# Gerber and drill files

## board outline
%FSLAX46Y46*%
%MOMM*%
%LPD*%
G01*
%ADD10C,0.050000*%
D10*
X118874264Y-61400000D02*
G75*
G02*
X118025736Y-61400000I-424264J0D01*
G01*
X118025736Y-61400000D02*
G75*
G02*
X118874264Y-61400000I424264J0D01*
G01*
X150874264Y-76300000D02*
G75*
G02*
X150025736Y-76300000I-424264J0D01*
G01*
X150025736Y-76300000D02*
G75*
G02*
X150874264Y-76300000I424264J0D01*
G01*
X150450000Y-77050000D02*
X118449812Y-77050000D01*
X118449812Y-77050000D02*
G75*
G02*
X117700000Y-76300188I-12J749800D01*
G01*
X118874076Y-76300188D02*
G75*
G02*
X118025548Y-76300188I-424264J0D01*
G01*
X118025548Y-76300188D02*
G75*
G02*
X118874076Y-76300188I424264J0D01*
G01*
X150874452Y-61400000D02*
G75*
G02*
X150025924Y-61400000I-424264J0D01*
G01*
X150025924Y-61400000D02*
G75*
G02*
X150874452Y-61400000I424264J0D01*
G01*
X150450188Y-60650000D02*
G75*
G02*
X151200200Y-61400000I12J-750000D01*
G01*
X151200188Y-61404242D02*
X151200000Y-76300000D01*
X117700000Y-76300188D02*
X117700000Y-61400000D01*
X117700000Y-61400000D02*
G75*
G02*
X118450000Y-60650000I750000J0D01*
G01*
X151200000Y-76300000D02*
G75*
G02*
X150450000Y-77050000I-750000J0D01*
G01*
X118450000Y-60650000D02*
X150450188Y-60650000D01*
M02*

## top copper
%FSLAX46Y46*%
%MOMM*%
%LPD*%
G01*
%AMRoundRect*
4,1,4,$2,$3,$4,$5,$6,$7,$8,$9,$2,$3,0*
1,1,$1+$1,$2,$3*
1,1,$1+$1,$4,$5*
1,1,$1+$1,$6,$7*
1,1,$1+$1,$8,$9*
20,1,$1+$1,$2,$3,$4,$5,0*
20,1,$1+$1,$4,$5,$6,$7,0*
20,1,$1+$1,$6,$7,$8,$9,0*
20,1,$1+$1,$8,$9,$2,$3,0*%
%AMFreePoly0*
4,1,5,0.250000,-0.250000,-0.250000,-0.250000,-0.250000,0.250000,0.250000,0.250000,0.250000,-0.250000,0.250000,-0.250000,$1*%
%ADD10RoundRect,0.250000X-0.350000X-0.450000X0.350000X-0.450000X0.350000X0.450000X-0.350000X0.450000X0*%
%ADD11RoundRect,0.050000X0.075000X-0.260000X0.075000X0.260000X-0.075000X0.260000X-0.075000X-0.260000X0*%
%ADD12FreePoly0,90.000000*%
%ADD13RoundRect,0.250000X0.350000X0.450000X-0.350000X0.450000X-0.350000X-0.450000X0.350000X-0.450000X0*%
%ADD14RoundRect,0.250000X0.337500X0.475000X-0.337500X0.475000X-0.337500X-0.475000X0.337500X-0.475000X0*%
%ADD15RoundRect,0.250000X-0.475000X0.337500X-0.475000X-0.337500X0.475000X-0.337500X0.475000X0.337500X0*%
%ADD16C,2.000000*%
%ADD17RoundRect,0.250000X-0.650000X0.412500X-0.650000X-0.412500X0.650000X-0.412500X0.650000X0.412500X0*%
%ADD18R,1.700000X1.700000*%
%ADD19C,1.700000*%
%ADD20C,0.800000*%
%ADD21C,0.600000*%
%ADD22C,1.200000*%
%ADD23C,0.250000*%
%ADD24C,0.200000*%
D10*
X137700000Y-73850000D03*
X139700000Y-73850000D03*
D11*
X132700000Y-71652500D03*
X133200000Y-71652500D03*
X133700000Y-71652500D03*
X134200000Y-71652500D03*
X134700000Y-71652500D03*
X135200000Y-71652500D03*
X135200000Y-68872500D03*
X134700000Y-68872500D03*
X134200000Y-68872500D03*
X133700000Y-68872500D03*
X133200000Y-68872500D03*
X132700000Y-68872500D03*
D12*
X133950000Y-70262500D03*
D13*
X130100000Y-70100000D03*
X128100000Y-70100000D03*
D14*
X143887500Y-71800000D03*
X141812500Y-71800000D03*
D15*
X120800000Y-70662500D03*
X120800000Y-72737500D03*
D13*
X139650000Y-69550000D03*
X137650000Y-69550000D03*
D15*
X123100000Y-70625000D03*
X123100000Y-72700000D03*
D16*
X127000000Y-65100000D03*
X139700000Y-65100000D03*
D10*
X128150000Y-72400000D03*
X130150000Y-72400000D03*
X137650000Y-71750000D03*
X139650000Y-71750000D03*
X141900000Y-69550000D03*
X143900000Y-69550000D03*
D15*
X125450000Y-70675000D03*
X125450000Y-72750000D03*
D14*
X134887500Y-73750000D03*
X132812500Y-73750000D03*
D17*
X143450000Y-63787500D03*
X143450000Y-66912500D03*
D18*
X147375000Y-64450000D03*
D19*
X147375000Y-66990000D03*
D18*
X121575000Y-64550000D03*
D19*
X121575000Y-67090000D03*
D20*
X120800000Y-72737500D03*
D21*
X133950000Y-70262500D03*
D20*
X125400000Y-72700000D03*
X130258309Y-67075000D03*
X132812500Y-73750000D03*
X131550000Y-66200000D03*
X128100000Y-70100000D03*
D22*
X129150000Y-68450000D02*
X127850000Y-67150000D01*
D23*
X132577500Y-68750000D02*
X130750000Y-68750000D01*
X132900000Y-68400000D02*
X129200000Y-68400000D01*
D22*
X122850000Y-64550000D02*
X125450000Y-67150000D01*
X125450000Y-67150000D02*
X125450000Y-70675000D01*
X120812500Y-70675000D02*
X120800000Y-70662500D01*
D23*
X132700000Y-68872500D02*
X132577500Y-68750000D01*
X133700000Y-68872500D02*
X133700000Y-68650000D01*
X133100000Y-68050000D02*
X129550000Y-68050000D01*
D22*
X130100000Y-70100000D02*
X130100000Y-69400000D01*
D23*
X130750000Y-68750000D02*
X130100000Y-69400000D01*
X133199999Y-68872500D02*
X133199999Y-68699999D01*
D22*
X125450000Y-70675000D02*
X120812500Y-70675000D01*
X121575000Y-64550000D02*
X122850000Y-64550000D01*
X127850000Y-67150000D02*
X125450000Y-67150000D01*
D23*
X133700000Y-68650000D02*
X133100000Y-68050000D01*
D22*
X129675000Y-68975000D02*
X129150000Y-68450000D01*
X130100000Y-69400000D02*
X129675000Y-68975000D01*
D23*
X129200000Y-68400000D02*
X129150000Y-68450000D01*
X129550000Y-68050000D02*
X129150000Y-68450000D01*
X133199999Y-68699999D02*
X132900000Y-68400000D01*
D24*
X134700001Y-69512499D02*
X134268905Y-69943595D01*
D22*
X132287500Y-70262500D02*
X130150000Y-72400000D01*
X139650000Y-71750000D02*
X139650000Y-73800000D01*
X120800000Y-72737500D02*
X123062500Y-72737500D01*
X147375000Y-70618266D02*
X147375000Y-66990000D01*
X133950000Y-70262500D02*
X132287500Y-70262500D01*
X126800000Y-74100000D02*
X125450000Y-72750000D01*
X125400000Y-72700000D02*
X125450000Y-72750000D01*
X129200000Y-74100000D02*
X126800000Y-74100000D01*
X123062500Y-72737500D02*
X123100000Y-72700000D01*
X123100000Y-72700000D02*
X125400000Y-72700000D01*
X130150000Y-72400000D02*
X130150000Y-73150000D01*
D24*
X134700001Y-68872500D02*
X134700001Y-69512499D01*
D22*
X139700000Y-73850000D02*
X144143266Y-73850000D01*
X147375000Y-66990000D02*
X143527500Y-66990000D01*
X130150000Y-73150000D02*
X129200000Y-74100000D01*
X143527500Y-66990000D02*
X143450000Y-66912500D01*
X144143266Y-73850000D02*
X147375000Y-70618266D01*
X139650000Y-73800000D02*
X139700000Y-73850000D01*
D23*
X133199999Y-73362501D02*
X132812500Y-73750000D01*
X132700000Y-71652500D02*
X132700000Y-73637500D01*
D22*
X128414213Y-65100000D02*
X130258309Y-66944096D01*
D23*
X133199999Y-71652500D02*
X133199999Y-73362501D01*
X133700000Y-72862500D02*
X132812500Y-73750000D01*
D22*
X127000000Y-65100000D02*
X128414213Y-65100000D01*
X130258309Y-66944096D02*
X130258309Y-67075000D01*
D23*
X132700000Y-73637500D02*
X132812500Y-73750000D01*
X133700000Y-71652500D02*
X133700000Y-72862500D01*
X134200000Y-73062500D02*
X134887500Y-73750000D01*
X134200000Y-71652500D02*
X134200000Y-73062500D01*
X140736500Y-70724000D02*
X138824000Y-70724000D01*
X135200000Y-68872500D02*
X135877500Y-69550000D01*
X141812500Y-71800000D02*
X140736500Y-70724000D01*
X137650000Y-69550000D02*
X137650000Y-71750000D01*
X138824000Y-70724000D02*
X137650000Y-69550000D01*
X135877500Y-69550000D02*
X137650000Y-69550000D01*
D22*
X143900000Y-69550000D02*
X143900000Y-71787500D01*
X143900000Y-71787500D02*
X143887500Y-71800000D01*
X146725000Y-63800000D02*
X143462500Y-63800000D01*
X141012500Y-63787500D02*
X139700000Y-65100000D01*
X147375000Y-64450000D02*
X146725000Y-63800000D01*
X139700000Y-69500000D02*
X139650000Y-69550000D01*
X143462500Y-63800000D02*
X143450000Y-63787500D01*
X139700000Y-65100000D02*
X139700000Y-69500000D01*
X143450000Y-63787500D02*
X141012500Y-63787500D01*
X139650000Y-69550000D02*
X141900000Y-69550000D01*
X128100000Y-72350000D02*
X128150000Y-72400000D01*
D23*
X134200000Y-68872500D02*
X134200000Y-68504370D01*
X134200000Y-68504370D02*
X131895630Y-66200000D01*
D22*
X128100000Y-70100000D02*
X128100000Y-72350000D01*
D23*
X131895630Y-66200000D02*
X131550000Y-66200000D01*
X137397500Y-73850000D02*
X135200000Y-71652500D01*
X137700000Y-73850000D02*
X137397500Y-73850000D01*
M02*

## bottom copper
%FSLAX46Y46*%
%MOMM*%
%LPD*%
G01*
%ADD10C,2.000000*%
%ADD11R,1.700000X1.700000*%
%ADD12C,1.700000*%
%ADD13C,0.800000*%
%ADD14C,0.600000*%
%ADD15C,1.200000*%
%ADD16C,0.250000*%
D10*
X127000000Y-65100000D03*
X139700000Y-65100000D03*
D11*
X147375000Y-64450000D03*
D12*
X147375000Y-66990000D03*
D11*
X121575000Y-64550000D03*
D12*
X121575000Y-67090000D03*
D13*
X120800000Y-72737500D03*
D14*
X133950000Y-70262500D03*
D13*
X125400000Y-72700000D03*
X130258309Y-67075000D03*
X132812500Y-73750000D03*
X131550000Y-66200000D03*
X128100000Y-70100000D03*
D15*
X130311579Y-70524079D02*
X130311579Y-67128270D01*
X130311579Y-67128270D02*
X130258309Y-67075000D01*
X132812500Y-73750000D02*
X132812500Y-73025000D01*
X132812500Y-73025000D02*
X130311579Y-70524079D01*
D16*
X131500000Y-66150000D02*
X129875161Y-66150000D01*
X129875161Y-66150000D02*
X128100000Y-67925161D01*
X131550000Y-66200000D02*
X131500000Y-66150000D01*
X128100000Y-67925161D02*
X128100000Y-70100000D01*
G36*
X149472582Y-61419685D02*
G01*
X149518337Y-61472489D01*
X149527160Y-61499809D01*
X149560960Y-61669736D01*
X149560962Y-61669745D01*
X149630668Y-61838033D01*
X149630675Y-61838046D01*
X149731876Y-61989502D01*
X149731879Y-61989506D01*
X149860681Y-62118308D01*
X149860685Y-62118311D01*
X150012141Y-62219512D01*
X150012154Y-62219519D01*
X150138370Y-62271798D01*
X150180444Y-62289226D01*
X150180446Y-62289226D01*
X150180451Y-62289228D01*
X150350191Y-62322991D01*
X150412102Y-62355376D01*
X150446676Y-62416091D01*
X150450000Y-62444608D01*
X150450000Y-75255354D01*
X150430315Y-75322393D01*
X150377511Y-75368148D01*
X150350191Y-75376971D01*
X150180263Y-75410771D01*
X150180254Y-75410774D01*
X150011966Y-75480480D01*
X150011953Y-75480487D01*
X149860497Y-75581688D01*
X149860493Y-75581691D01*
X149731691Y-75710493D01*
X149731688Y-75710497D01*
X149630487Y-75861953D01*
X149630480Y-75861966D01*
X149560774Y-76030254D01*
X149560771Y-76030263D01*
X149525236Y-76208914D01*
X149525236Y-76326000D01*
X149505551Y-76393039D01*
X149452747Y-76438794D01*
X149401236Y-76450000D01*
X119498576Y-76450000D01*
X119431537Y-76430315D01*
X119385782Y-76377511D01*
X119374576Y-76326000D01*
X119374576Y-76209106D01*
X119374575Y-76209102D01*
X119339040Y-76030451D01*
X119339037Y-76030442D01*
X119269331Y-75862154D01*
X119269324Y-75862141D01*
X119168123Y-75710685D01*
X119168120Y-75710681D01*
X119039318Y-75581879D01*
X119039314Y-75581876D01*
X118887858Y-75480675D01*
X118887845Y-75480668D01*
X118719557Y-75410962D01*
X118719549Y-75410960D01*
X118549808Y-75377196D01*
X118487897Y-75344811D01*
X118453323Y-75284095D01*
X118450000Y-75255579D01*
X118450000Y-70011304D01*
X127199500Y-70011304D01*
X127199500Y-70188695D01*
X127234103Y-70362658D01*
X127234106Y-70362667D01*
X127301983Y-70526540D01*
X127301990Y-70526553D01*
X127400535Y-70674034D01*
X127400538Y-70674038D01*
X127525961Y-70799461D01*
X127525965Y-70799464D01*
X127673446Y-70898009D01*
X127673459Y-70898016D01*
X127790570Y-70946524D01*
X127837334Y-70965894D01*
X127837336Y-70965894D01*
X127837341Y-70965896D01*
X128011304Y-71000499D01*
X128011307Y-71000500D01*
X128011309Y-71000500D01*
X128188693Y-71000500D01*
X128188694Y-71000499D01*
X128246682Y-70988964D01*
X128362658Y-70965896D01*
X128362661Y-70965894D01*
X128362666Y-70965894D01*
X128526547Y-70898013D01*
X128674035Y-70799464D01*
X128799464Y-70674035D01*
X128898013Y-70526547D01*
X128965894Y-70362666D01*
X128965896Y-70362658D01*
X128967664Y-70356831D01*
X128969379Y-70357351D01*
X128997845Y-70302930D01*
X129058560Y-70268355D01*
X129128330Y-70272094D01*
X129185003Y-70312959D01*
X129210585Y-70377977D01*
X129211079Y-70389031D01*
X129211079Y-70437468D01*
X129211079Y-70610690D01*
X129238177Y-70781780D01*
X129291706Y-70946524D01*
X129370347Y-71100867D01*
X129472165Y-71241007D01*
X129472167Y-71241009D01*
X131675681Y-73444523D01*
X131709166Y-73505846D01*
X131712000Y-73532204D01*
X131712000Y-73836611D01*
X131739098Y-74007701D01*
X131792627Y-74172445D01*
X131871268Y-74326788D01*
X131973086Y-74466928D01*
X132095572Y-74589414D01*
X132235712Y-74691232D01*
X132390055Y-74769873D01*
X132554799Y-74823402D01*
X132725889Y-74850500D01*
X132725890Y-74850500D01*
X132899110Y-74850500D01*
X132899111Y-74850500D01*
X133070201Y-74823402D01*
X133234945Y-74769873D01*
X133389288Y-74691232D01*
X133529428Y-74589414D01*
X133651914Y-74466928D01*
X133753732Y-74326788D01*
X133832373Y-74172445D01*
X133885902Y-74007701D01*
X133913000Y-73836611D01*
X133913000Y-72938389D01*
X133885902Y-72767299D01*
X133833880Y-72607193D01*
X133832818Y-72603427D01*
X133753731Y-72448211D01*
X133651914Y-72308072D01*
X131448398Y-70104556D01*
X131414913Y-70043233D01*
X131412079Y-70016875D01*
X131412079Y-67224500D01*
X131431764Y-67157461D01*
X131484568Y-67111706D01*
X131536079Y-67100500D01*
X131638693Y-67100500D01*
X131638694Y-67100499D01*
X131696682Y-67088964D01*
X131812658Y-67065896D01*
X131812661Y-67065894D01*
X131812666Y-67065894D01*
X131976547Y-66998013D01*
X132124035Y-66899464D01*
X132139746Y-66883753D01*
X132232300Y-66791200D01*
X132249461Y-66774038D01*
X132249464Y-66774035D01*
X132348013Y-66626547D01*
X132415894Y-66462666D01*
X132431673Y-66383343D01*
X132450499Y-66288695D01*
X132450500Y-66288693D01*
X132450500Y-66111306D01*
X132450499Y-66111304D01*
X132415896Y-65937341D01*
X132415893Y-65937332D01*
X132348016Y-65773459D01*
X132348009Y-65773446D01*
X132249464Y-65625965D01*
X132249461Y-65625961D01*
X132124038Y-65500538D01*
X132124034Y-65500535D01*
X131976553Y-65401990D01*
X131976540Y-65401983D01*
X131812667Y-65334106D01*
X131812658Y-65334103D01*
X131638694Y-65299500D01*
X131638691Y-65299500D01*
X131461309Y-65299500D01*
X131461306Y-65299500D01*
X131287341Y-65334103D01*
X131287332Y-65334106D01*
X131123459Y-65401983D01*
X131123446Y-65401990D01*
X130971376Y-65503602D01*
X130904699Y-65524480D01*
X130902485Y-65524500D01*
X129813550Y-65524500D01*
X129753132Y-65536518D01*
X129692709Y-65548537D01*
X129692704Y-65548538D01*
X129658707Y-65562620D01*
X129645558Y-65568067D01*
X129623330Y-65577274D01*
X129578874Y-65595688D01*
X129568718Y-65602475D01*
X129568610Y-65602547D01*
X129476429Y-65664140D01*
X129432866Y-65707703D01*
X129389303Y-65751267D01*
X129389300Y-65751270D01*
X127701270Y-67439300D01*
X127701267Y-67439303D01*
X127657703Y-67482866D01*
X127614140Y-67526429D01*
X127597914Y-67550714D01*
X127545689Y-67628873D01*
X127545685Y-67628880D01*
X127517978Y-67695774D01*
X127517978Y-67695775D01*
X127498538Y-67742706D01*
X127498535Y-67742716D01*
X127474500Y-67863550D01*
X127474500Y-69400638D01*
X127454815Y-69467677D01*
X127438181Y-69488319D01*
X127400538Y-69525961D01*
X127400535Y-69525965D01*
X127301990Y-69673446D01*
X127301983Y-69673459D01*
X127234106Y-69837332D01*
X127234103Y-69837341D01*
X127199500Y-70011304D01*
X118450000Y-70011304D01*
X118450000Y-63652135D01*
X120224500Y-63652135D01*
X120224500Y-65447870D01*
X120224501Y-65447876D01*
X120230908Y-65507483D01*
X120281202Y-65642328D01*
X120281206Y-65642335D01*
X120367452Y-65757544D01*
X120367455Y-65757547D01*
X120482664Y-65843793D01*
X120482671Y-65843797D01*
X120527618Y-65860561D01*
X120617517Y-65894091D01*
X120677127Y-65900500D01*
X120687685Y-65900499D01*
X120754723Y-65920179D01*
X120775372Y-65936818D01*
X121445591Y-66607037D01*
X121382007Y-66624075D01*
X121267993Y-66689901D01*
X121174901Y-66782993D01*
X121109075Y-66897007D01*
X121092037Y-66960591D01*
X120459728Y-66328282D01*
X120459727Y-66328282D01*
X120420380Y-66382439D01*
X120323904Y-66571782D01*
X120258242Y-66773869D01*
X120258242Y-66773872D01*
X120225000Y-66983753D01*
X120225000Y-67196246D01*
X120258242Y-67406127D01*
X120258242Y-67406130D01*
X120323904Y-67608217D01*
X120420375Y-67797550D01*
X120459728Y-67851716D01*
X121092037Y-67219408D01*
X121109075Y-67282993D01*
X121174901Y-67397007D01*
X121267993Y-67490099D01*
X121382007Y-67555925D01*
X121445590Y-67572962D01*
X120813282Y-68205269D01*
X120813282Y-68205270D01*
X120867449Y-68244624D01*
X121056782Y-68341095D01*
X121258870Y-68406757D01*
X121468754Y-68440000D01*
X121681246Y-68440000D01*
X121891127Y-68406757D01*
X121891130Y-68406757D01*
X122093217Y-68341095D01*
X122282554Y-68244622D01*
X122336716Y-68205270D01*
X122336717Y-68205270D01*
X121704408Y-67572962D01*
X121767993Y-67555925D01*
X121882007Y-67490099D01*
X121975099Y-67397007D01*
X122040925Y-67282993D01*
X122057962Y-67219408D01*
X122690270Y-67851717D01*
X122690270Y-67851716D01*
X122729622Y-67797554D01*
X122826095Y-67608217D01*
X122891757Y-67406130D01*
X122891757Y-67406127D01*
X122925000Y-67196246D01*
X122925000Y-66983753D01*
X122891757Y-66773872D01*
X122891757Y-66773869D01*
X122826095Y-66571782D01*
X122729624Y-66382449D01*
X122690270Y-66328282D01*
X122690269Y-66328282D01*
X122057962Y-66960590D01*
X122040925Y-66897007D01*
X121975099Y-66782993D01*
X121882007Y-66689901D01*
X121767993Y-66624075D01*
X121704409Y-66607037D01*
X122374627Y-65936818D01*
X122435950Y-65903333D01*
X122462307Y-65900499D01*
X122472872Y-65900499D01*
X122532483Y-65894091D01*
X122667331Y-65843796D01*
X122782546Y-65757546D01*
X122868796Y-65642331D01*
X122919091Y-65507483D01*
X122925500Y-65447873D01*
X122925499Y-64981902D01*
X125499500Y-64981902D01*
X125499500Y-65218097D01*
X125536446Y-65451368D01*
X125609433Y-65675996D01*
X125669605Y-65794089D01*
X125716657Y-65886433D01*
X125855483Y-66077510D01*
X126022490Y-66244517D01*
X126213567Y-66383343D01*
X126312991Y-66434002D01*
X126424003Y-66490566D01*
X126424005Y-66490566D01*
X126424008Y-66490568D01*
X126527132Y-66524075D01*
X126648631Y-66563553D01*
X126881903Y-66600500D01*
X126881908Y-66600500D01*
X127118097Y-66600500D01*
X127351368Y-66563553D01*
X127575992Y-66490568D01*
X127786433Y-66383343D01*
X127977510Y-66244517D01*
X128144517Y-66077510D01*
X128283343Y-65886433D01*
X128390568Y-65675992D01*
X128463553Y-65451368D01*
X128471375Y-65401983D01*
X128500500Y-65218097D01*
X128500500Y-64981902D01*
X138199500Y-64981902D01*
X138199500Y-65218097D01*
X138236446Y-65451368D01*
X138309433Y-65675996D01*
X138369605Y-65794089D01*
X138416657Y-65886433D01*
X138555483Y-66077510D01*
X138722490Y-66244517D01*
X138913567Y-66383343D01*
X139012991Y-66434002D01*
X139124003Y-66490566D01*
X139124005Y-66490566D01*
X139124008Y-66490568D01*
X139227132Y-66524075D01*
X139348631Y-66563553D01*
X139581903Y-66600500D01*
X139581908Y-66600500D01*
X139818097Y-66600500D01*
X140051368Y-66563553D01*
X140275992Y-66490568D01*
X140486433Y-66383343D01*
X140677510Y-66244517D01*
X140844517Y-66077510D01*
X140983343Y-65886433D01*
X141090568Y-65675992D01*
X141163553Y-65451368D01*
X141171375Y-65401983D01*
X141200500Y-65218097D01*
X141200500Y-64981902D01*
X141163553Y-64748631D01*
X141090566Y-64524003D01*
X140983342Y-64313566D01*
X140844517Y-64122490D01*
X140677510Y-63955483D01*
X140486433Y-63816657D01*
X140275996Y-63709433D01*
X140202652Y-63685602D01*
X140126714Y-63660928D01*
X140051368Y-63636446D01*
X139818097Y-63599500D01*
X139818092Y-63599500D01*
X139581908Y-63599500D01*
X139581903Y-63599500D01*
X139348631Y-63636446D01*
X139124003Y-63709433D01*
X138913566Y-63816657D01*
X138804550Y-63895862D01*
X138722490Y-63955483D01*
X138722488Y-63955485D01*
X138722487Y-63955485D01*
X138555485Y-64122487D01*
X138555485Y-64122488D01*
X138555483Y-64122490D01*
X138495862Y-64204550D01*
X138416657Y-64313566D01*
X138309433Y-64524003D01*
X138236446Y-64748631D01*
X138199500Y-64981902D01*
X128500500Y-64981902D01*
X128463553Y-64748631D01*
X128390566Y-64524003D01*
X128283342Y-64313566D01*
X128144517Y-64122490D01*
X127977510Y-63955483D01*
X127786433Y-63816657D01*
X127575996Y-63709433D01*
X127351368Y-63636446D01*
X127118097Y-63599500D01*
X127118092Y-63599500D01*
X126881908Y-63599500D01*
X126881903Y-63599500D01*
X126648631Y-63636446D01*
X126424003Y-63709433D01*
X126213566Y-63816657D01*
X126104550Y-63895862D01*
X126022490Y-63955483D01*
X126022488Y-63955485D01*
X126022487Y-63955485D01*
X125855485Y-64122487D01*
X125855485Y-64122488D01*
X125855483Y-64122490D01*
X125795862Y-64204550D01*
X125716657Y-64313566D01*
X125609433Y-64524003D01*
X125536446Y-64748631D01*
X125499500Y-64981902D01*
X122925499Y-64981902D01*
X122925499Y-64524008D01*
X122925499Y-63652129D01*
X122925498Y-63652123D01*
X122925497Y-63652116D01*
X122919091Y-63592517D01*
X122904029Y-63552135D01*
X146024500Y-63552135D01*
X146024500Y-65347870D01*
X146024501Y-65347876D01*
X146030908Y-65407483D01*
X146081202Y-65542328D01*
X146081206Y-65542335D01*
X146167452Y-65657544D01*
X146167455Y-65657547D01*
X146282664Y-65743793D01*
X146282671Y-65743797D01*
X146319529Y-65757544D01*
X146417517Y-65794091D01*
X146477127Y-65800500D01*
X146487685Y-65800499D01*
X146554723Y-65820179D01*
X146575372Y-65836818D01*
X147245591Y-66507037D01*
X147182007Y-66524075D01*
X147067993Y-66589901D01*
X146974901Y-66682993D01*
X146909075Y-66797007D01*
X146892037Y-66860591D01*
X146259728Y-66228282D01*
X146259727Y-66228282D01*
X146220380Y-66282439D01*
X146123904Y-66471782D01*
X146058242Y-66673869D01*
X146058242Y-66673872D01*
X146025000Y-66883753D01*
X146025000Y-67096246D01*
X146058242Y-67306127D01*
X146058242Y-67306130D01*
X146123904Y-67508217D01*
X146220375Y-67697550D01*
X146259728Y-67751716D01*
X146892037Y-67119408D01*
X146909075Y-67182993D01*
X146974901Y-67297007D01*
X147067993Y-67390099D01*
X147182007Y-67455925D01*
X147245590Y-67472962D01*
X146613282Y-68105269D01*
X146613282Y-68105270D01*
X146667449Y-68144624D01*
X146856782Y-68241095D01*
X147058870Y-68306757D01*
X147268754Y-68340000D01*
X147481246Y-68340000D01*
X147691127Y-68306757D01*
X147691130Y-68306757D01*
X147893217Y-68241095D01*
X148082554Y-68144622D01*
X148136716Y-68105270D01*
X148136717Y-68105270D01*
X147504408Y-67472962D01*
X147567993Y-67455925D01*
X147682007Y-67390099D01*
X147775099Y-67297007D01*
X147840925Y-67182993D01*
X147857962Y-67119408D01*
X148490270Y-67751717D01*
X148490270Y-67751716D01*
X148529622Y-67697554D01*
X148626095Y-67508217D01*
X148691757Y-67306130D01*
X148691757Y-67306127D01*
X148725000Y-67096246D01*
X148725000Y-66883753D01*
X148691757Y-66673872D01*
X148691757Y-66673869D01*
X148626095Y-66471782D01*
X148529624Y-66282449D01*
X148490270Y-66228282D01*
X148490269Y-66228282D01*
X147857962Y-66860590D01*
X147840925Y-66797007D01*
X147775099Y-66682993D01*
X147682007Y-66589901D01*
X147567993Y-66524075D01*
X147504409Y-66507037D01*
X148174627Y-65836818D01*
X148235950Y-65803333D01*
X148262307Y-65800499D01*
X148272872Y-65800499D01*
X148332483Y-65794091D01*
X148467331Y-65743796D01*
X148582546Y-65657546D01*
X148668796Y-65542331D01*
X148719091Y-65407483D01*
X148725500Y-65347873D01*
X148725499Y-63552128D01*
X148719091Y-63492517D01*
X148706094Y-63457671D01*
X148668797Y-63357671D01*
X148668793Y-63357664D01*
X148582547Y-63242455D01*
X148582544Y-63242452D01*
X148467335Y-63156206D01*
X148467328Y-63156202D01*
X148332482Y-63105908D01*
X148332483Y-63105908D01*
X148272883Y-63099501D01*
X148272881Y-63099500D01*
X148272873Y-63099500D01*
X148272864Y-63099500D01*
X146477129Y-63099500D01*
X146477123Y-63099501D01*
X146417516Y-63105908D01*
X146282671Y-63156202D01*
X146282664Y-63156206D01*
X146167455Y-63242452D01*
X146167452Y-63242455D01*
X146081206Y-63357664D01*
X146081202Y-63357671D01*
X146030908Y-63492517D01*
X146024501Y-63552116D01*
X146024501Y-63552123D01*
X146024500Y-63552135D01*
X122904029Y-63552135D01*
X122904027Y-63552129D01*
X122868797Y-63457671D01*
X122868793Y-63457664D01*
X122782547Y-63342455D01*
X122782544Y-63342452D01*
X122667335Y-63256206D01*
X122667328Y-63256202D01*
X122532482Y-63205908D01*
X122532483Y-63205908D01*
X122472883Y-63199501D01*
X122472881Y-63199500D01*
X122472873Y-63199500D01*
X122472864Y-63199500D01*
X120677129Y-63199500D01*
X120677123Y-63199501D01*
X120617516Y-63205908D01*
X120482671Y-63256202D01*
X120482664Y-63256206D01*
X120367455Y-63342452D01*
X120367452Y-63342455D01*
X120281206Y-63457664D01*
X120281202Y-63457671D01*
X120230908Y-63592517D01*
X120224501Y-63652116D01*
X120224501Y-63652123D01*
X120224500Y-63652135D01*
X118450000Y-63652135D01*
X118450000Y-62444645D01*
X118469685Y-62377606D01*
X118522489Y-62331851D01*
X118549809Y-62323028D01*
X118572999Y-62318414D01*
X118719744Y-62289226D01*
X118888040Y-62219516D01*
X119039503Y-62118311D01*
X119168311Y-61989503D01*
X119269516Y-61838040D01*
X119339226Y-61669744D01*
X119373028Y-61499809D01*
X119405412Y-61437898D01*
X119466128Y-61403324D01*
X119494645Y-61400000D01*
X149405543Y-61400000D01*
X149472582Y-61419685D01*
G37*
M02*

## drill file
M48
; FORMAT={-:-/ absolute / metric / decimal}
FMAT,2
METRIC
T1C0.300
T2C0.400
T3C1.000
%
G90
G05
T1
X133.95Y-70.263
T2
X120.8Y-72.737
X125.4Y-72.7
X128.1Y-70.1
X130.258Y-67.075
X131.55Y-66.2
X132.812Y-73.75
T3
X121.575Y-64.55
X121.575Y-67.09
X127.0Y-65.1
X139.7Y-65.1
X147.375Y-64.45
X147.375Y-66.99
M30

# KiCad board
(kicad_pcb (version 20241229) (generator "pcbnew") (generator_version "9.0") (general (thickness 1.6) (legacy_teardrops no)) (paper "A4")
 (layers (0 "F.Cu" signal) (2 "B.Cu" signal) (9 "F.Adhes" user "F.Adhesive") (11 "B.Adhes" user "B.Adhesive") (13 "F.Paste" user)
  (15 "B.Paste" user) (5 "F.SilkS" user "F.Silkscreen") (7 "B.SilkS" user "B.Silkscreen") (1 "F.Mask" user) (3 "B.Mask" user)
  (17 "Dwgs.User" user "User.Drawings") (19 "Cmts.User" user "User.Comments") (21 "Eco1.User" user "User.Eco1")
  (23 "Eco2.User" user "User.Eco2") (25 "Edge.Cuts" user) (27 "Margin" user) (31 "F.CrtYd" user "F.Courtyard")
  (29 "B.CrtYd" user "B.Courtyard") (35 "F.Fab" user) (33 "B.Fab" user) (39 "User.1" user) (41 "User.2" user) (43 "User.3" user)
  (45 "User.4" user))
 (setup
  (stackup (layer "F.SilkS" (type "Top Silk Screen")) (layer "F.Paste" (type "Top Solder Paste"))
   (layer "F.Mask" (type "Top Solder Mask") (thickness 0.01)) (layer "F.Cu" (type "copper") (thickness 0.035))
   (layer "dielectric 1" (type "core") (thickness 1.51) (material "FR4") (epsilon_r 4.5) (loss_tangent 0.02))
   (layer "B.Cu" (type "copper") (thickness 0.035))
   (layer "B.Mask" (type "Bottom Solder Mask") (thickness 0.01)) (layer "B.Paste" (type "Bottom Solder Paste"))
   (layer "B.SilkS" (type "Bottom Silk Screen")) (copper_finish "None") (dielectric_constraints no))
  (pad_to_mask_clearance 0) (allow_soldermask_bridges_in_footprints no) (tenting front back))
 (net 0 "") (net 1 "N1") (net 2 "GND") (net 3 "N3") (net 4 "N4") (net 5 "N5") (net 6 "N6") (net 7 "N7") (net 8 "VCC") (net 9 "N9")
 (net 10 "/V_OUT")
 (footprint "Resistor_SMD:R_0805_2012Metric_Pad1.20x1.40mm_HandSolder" (layer "F.Cu") (at 138.7 73.85)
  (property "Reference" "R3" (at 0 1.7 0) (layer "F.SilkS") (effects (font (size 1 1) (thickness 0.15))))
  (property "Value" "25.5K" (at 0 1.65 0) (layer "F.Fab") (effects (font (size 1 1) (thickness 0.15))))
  (pad "1" smd roundrect (at -1 0) (size 1.2 1.4) (layers "F.Cu" "F.Mask" "F.Paste") (roundrect_rratio 0.208333) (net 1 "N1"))
  (pad "2" smd roundrect (at 1 0) (size 1.2 1.4) (layers "F.Cu" "F.Mask" "F.Paste") (roundrect_rratio 0.208333) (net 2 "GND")))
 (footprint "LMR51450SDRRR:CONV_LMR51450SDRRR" (layer "F.Cu") (at 133.95 70.2625 90)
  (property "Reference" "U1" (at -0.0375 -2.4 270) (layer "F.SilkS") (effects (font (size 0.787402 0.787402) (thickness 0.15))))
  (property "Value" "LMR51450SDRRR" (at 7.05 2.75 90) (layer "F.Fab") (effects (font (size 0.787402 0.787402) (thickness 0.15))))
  (pad "1" smd roundrect (at -1.39 -1.25 90) (size 0.62 0.25) (layers "F.Cu" "F.Paste") (roundrect_rratio 0.2) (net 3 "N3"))
  (pad "2" smd roundrect (at -1.39 -0.75 90) (size 0.62 0.25) (layers "F.Cu" "F.Paste") (roundrect_rratio 0.2) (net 3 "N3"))
  (pad "3" smd roundrect (at -1.39 -0.25 90) (size 0.62 0.25) (layers "F.Cu" "F.Paste") (roundrect_rratio 0.2) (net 3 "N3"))
  (pad "4" smd roundrect (at -1.39 0.25 90) (size 0.62 0.25) (layers "F.Cu" "F.Paste") (roundrect_rratio 0.2) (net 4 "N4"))
  (pad "5" smd roundrect (at -1.39 0.75 90) (size 0.62 0.25) (layers "F.Cu" "F.Paste") (roundrect_rratio 0.2) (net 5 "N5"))
  (pad "6" smd roundrect (at -1.39 1.25 90) (size 0.62 0.25) (layers "F.Cu" "F.Paste") (roundrect_rratio 0.2) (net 1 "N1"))
  (pad "7" smd roundrect (at 1.39 1.25 90) (size 0.62 0.25) (layers "F.Cu" "F.Paste") (roundrect_rratio 0.2) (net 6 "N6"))
  (pad "8" smd roundrect (at 1.39 0.75 90) (size 0.62 0.25) (layers "F.Cu" "F.Paste") (roundrect_rratio 0.2) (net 2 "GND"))
  (pad "9" smd roundrect (at 1.39 0.25 90) (size 0.62 0.25) (layers "F.Cu" "F.Paste") (roundrect_rratio 0.2) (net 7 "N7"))
  (pad "10" smd roundrect (at 1.39 -0.25 90) (size 0.62 0.25) (layers "F.Cu" "F.Paste") (roundrect_rratio 0.2) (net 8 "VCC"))
  (pad "11" smd roundrect (at 1.39 -0.75 90) (size 0.62 0.25) (layers "F.Cu" "F.Paste") (roundrect_rratio 0.2) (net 8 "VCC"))
  (pad "12" smd roundrect (at 1.39 -1.25 90) (size 0.62 0.25) (layers "F.Cu" "F.Paste") (roundrect_rratio 0.2) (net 8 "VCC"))
  (pad "13" smd custom (at 0 0 90) (size 0.5 0.5) (layers "F.Cu") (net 2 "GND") (options (clearance outline) (anchor rect)) (primitives)))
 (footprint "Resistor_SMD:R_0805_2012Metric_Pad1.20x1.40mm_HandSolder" (layer "F.Cu") (at 129.1 70.1 180)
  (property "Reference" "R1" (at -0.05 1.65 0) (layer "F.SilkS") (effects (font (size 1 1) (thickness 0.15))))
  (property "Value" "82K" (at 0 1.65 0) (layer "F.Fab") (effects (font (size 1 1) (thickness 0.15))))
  (pad "1" smd roundrect (at -1 0 180) (size 1.2 1.4) (layers "F.Cu" "F.Mask" "F.Paste") (roundrect_rratio 0.208333) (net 8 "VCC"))
  (pad "2" smd roundrect (at 1 0 180) (size 1.2 1.4) (layers "F.Cu" "F.Mask" "F.Paste") (roundrect_rratio 0.208333) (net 7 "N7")))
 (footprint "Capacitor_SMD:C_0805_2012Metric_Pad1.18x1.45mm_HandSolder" (layer "F.Cu") (at 142.85 71.8 180)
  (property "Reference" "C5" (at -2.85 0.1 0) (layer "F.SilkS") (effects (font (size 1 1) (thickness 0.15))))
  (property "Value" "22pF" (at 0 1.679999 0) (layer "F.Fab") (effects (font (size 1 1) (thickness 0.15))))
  (pad "1" smd roundrect (at -1.0375 0 180) (size 1.175 1.45) (layers "F.Cu" "F.Mask" "F.Paste") (roundrect_rratio 0.212766) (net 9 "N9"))
  (pad "2" smd roundrect (at 1.0375 0 180) (size 1.175 1.45) (layers "F.Cu" "F.Mask" "F.Paste") (roundrect_rratio 0.212766) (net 6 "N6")))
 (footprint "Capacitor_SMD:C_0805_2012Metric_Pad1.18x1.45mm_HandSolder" (layer "F.Cu") (at 120.8 71.7 -90)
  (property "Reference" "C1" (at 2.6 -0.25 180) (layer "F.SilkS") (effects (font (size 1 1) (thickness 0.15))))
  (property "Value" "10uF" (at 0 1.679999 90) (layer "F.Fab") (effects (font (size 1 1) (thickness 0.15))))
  (pad "1" smd roundrect (at -1.0375 0 270) (size 1.175 1.45) (layers "F.Cu" "F.Mask" "F.Paste") (roundrect_rratio 0.212766) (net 8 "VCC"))
  (pad "2" smd roundrect (at 1.0375 0 270) (size 1.175 1.45) (layers "F.Cu" "F.Mask" "F.Paste") (roundrect_rratio 0.212766) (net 2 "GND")))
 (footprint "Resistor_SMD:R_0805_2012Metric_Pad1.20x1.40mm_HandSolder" (layer "F.Cu") (at 138.65 69.55 180)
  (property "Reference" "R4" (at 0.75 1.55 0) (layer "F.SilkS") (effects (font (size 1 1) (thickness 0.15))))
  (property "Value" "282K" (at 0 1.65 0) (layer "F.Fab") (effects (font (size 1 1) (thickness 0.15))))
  (pad "1" smd roundrect (at -1 0 180) (size 1.2 1.4) (layers "F.Cu" "F.Mask" "F.Paste") (roundrect_rratio 0.208333) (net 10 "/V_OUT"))
  (pad "2" smd roundrect (at 1 0 180) (size 1.2 1.4) (layers "F.Cu" "F.Mask" "F.Paste") (roundrect_rratio 0.208333) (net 6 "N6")))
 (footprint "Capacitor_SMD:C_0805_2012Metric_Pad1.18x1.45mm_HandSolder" (layer "F.Cu") (at 123.1 71.6625 -90)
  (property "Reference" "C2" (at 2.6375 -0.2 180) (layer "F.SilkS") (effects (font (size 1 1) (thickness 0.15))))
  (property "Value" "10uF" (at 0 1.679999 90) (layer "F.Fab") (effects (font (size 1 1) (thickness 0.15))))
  (pad "1" smd roundrect (at -1.0375 0 270) (size 1.175 1.45) (layers "F.Cu" "F.Mask" "F.Paste") (roundrect_rratio 0.212766) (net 8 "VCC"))
  (pad "2" smd roundrect (at 1.0375 0 270) (size 1.175 1.45) (layers "F.Cu" "F.Mask" "F.Paste") (roundrect_rratio 0.212766) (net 2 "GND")))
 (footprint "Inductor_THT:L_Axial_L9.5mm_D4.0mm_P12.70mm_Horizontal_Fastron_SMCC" (layer "F.Cu") (at 127 65.1)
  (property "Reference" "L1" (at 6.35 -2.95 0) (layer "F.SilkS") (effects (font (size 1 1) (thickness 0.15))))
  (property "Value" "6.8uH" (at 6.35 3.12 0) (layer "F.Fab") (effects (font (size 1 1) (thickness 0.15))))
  (pad "1" thru_hole circle (at 0 0) (size 2 2) (drill 1) (layers "*.Cu" "*.Mask") (remove_unused_layers no) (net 3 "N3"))
  (pad "2" thru_hole circle (at 12.7 0) (size 2 2) (drill 1) (layers "*.Cu" "*.Mask") (remove_unused_layers no) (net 10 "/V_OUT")))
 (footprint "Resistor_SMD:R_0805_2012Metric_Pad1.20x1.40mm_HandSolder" (layer "F.Cu") (at 129.15 72.4)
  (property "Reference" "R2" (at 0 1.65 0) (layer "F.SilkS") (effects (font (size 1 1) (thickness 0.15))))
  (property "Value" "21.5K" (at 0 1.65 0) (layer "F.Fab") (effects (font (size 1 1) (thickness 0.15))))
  (pad "1" smd roundrect (at -1 0) (size 1.2 1.4) (layers "F.Cu" "F.Mask" "F.Paste") (roundrect_rratio 0.208333) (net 7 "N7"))
  (pad "2" smd roundrect (at 1 0) (size 1.2 1.4) (layers "F.Cu" "F.Mask" "F.Paste") (roundrect_rratio 0.208333) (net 2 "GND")))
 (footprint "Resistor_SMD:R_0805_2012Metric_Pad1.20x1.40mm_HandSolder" (layer "F.Cu") (at 138.65 71.75)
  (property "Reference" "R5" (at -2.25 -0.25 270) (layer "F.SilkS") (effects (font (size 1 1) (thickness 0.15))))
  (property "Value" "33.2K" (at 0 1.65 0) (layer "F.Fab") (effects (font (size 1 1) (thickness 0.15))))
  (pad "1" smd roundrect (at -1 0) (size 1.2 1.4) (layers "F.Cu" "F.Mask" "F.Paste") (roundrect_rratio 0.208333) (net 6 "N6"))
  (pad "2" smd roundrect (at 1 0) (size 1.2 1.4) (layers "F.Cu" "F.Mask" "F.Paste") (roundrect_rratio 0.208333) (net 2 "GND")))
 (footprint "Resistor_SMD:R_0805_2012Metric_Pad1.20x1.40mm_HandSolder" (layer "F.Cu") (at 142.9 69.55)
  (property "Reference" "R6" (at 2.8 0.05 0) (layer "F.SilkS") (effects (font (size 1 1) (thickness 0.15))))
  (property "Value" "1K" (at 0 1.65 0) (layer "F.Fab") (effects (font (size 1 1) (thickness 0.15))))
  (pad "1" smd roundrect (at -1 0) (size 1.2 1.4) (layers "F.Cu" "F.Mask" "F.Paste") (roundrect_rratio 0.208333) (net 10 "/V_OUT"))
  (pad "2" smd roundrect (at 1 0) (size 1.2 1.4) (layers "F.Cu" "F.Mask" "F.Paste") (roundrect_rratio 0.208333) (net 9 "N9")))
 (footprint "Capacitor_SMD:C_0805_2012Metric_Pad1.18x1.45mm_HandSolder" (layer "F.Cu") (at 125.45 71.7125 -90)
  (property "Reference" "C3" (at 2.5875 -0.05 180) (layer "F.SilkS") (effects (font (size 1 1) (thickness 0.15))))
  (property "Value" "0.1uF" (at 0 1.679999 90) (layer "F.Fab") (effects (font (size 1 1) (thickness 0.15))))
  (pad "1" smd roundrect (at -1.0375 0 270) (size 1.175 1.45) (layers "F.Cu" "F.Mask" "F.Paste") (roundrect_rratio 0.212766) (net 8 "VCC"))
  (pad "2" smd roundrect (at 1.0375 0 270) (size 1.175 1.45) (layers "F.Cu" "F.Mask" "F.Paste") (roundrect_rratio 0.212766) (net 2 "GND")))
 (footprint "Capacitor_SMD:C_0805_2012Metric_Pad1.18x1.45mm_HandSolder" (layer "F.Cu") (at 133.85 73.75 180)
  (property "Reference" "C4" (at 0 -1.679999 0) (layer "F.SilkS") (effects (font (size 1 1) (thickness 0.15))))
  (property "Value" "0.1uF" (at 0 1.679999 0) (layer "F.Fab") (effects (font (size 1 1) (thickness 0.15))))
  (pad "1" smd roundrect (at -1.0375 0 180) (size 1.175 1.45) (layers "F.Cu" "F.Mask" "F.Paste") (roundrect_rratio 0.212766) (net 4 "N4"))
  (pad "2" smd roundrect (at 1.0375 0 180) (size 1.175 1.45) (layers "F.Cu" "F.Mask" "F.Paste") (roundrect_rratio 0.212766) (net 3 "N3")))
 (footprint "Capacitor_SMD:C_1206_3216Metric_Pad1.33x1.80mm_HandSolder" (layer "F.Cu") (at 143.45 65.35 -90)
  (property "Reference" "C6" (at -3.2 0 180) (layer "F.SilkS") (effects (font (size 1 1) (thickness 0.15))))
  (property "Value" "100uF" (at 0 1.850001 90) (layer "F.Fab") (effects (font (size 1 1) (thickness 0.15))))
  (pad "1" smd roundrect (at -1.5625 0 270) (size 1.325 1.8) (layers "F.Cu" "F.Mask" "F.Paste") (roundrect_rratio 0.188679)
   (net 10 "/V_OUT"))
  (pad "2" smd roundrect (at 1.5625 0 270) (size 1.325 1.8) (layers "F.Cu" "F.Mask" "F.Paste") (roundrect_rratio 0.188679) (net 2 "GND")))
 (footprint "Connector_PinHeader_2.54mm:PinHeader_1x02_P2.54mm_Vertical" (layer "F.Cu") (at 147.375 64.45)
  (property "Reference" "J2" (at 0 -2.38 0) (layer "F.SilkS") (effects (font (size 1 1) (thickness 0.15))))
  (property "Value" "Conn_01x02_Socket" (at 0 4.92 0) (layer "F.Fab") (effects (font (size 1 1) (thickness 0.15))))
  (pad "1" thru_hole rect (at 0 0) (size 1.7 1.7) (drill 1) (layers "*.Cu" "*.Mask") (remove_unused_layers no) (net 10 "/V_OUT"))
  (pad "2" thru_hole circle (at 0 2.54) (size 1.7 1.7) (drill 1) (layers "*.Cu" "*.Mask") (remove_unused_layers no) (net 2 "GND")))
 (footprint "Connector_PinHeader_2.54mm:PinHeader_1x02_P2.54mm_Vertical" (layer "F.Cu") (at 121.575 64.55)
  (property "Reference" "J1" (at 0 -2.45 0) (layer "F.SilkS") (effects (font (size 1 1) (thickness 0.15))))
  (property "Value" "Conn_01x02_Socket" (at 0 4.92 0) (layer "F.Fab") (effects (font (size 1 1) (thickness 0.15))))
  (pad "1" thru_hole rect (at 0 0) (size 1.7 1.7) (drill 1) (layers "*.Cu" "*.Mask") (remove_unused_layers no) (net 8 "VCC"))
  (pad "2" thru_hole circle (at 0 2.54) (size 1.7 1.7) (drill 1) (layers "*.Cu" "*.Mask") (remove_unused_layers no) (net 2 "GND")))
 (gr_circle (center 118.45 61.4) (end 118.75 61.7) (stroke (width 0.05) (type default)) (fill no) (layer "Edge.Cuts"))
 (gr_circle (center 150.45 76.3) (end 150.75 76.6) (stroke (width 0.05) (type default)) (fill no) (layer "Edge.Cuts"))
 (gr_line (start 150.45 77.05) (end 118.449812 77.05) (stroke (width 0.05) (type default)) (layer "Edge.Cuts"))
 (gr_arc (start 118.449812 77.05) (mid 117.919615 76.830385) (end 117.7 76.300188) (stroke (width 0.05) (type default)) (layer "Edge.Cuts"))
 (gr_circle (center 118.449812 76.300188) (end 118.749812 76.600188) (stroke (width 0.05) (type default)) (fill no) (layer "Edge.Cuts"))
 (gr_circle (center 150.450188 61.4) (end 150.750188 61.7) (stroke (width 0.05) (type default)) (fill no) (layer "Edge.Cuts"))
 (gr_arc (start 150.450188 60.65) (mid 150.980518 60.86967) (end 151.200188 61.4) (stroke (width 0.05) (type default)) (layer "Edge.Cuts"))
 (gr_line (start 151.200188 61.404242) (end 151.2 76.3) (stroke (width 0.05) (type default)) (layer "Edge.Cuts"))
 (gr_line (start 117.7 76.300188) (end 117.7 61.4) (stroke (width 0.05) (type default)) (layer "Edge.Cuts"))
 (gr_arc (start 117.7 61.4) (mid 117.91967 60.86967) (end 118.45 60.65) (stroke (width 0.05) (type default)) (layer "Edge.Cuts"))
 (gr_arc (start 151.2 76.3) (mid 150.98033 76.83033) (end 150.45 77.05) (stroke (width 0.05) (type default)) (layer "Edge.Cuts"))
 (gr_line (start 118.45 60.65) (end 150.450188 60.65) (stroke (width 0.05) (type default)) (layer "Edge.Cuts"))
 (segment (start 129.15 68.45) (end 127.85 67.15) (width 1.2) (layer "F.Cu") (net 8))
 (segment (start 132.5775 68.75) (end 130.75 68.75) (width 0.25) (layer "F.Cu") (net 8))
 (segment (start 132.9 68.4) (end 129.2 68.4) (width 0.25) (layer "F.Cu") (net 8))
 (segment (start 122.85 64.55) (end 125.45 67.15) (width 1.2) (layer "F.Cu") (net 8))
 (segment (start 125.45 67.15) (end 125.45 70.675) (width 1.2) (layer "F.Cu") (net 8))
 (segment (start 120.8125 70.675) (end 120.8 70.6625) (width 1.2) (layer "F.Cu") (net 8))
 (segment (start 132.7 68.8725) (end 132.5775 68.75) (width 0.25) (layer "F.Cu") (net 8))
 (segment (start 133.7 68.8725) (end 133.7 68.65) (width 0.25) (layer "F.Cu") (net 8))
 (segment (start 133.1 68.05) (end 129.55 68.05) (width 0.25) (layer "F.Cu") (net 8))
 (segment (start 130.1 70.1) (end 130.1 69.4) (width 1.2) (layer "F.Cu") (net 8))
 (segment (start 130.75 68.75) (end 130.1 69.4) (width 0.25) (layer "F.Cu") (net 8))
 (segment (start 133.199999 68.8725) (end 133.199999 68.699999) (width 0.25) (layer "F.Cu") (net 8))
 (segment (start 125.45 70.675) (end 120.8125 70.675) (width 1.2) (layer "F.Cu") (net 8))
 (segment (start 121.575 64.55) (end 122.85 64.55) (width 1.2) (layer "F.Cu") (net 8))
 (segment (start 127.85 67.15) (end 125.45 67.15) (width 1.2) (layer "F.Cu") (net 8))
 (segment (start 133.7 68.65) (end 133.1 68.05) (width 0.25) (layer "F.Cu") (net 8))
 (segment (start 129.675 68.975) (end 129.15 68.45) (width 1.2) (layer "F.Cu") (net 8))
 (segment (start 130.1 69.4) (end 129.675 68.975) (width 1.2) (layer "F.Cu") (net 8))
 (segment (start 129.2 68.4) (end 129.15 68.45) (width 0.25) (layer "F.Cu") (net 8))
 (segment (start 129.55 68.05) (end 129.15 68.45) (width 0.25) (layer "F.Cu") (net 8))
 (segment (start 133.199999 68.699999) (end 132.9 68.4) (width 0.25) (layer "F.Cu") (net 8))
 (segment (start 134.700001 69.512499) (end 134.268905 69.943595) (width 0.2) (layer "F.Cu") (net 2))
 (segment (start 132.2875 70.2625) (end 130.15 72.4) (width 1.2) (layer "F.Cu") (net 2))
 (segment (start 139.65 71.75) (end 139.65 73.8) (width 1.2) (layer "F.Cu") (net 2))
 (segment (start 120.8 72.7375) (end 123.0625 72.7375) (width 1.2) (layer "F.Cu") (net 2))
 (segment (start 147.375 70.618266) (end 147.375 66.99) (width 1.2) (layer "F.Cu") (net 2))
 (segment (start 133.95 70.2625) (end 132.2875 70.2625) (width 1.2) (layer "F.Cu") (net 2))
 (segment (start 126.8 74.1) (end 125.45 72.75) (width 1.2) (layer "F.Cu") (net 2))
 (segment (start 125.4 72.7) (end 125.45 72.75) (width 1.2) (layer "F.Cu") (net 2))
 (segment (start 129.2 74.1) (end 126.8 74.1) (width 1.2) (layer "F.Cu") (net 2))
 (segment (start 123.0625 72.7375) (end 123.1 72.7) (width 1.2) (layer "F.Cu") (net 2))
 (segment (start 123.1 72.7) (end 125.4 72.7) (width 1.2) (layer "F.Cu") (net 2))
 (segment (start 130.15 72.4) (end 130.15 73.15) (width 1.2) (layer "F.Cu") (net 2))
 (segment (start 134.700001 68.8725) (end 134.700001 69.512499) (width 0.2) (layer "F.Cu") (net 2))
 (segment (start 139.7 73.85) (end 144.143266 73.85) (width 1.2) (layer "F.Cu") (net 2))
 (segment (start 147.375 66.99) (end 143.5275 66.99) (width 1.2) (layer "F.Cu") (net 2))
 (segment (start 130.15 73.15) (end 129.2 74.1) (width 1.2) (layer "F.Cu") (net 2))
 (segment (start 143.5275 66.99) (end 143.45 66.9125) (width 1.2) (layer "F.Cu") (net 2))
 (segment (start 144.143266 73.85) (end 147.375 70.618266) (width 1.2) (layer "F.Cu") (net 2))
 (segment (start 139.65 73.8) (end 139.7 73.85) (width 1.2) (layer "F.Cu") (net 2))
 (via (at 120.8 72.7375) (size 0.8) (drill 0.4) (layers "F.Cu" "B.Cu") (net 2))
 (via (at 133.95 70.2625) (size 0.6) (drill 0.3) (layers "F.Cu" "B.Cu") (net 2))
 (via (at 125.4 72.7) (size 0.8) (drill 0.4) (layers "F.Cu" "B.Cu") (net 2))
 (segment (start 133.199999 73.362501) (end 132.8125 73.75) (width 0.25) (layer "F.Cu") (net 3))
 (segment (start 132.7 71.6525) (end 132.7 73.6375) (width 0.25) (layer "F.Cu") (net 3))
 (segment (start 128.414213 65.1) (end 130.258309 66.944096) (width 1.2) (layer "F.Cu") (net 3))
 (segment (start 133.199999 71.6525) (end 133.199999 73.362501) (width 0.25) (layer "F.Cu") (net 3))
 (segment (start 133.7 72.8625) (end 132.8125 73.75) (width 0.25) (layer "F.Cu") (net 3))
 (segment (start 127 65.1) (end 128.414213 65.1) (width 1.2) (layer "F.Cu") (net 3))
 (segment (start 130.258309 66.944096) (end 130.258309 67.075) (width 1.2) (layer "F.Cu") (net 3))
 (segment (start 132.7 73.6375) (end 132.8125 73.75) (width 0.25) (layer "F.Cu") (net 3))
 (segment (start 133.7 71.6525) (end 133.7 72.8625) (width 0.25) (layer "F.Cu") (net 3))
 (via (at 130.258309 67.075) (size 0.8) (drill 0.4) (layers "F.Cu" "B.Cu") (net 3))
 (via (at 132.8125 73.75) (size 0.8) (drill 0.4) (layers "F.Cu" "B.Cu") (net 3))
 (segment (start 130.311579 70.524079) (end 130.311579 67.12827) (width 1.2) (layer "B.Cu") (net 3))
 (segment (start 130.311579 67.12827) (end 130.258309 67.075) (width 1.2) (layer "B.Cu") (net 3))
 (segment (start 132.8125 73.75) (end 132.8125 73.025) (width 1.2) (layer "B.Cu") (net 3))
 (segment (start 132.8125 73.025) (end 130.311579 70.524079) (width 1.2) (layer "B.Cu") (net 3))
 (segment (start 134.2 73.0625) (end 134.8875 73.75) (width 0.25) (layer "F.Cu") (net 4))
 (segment (start 134.2 71.6525) (end 134.2 73.0625) (width 0.25) (layer "F.Cu") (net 4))
 (segment (start 140.7365 70.724) (end 138.824 70.724) (width 0.25) (layer "F.Cu") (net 6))
 (segment (start 135.2 68.8725) (end 135.8775 69.55) (width 0.25) (layer "F.Cu") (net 6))
 (segment (start 141.8125 71.8) (end 140.7365 70.724) (width 0.25) (layer "F.Cu") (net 6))
 (segment (start 137.65 69.55) (end 137.65 71.75) (width 0.25) (layer "F.Cu") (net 6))
 (segment (start 138.824 70.724) (end 137.65 69.55) (width 0.25) (layer "F.Cu") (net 6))
 (segment (start 135.8775 69.55) (end 137.65 69.55) (width 0.25) (layer "F.Cu") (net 6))
 (segment (start 143.9 69.55) (end 143.9 71.7875) (width 1.2) (layer "F.Cu") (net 9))
 (segment (start 143.9 71.7875) (end 143.8875 71.8) (width 1.2) (layer "F.Cu") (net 9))
 (segment (start 146.725 63.8) (end 143.4625 63.8) (width 1.2) (layer "F.Cu") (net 10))
 (segment (start 141.0125 63.7875) (end 139.7 65.1) (width 1.2) (layer "F.Cu") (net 10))
 (segment (start 147.375 64.45) (end 146.725 63.8) (width 1.2) (layer "F.Cu") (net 10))
 (segment (start 139.7 69.5) (end 139.65 69.55) (width 1.2) (layer "F.Cu") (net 10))
 (segment (start 143.4625 63.8) (end 143.45 63.7875) (width 1.2) (layer "F.Cu") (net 10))
 (segment (start 139.7 65.1) (end 139.7 69.5) (width 1.2) (layer "F.Cu") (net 10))
 (segment (start 143.45 63.7875) (end 141.0125 63.7875) (width 1.2) (layer "F.Cu") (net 10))
 (segment (start 139.65 69.55) (end 141.9 69.55) (width 1.2) (layer "F.Cu") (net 10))
 (segment (start 128.1 72.35) (end 128.15 72.4) (width 1.2) (layer "F.Cu") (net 7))
 (segment (start 134.2 68.8725) (end 134.2 68.50437) (width 0.25) (layer "F.Cu") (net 7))
 (segment (start 134.2 68.50437) (end 131.89563 66.2) (width 0.25) (layer "F.Cu") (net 7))
 (segment (start 128.1 70.1) (end 128.1 72.35) (width 1.2) (layer "F.Cu") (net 7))
 (segment (start 131.89563 66.2) (end 131.55 66.2) (width 0.25) (layer "F.Cu") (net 7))
 (via (at 131.55 66.2) (size 0.8) (drill 0.4) (layers "F.Cu" "B.Cu") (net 7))
 (via (at 128.1 70.1) (size 0.8) (drill 0.4) (layers "F.Cu" "B.Cu") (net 7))
 (segment (start 131.5 66.15) (end 129.875161 66.15) (width 0.25) (layer "B.Cu") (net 7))
 (segment (start 129.875161 66.15) (end 128.1 67.925161) (width 0.25) (layer "B.Cu") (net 7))
 (segment (start 131.55 66.2) (end 131.5 66.15) (width 0.25) (layer "B.Cu") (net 7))
 (segment (start 128.1 67.925161) (end 128.1 70.1) (width 0.25) (layer "B.Cu") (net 7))
 (segment (start 137.3975 73.85) (end 135.2 71.6525) (width 0.25) (layer "F.Cu") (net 1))
 (segment (start 137.7 73.85) (end 137.3975 73.85) (width 0.25) (layer "F.Cu") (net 1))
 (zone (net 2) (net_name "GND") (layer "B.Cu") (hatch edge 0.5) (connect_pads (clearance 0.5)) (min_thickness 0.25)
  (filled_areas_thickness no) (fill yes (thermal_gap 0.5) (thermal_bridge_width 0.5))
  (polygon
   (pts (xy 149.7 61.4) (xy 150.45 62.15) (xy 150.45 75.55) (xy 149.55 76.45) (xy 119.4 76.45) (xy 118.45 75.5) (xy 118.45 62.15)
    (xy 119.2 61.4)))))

